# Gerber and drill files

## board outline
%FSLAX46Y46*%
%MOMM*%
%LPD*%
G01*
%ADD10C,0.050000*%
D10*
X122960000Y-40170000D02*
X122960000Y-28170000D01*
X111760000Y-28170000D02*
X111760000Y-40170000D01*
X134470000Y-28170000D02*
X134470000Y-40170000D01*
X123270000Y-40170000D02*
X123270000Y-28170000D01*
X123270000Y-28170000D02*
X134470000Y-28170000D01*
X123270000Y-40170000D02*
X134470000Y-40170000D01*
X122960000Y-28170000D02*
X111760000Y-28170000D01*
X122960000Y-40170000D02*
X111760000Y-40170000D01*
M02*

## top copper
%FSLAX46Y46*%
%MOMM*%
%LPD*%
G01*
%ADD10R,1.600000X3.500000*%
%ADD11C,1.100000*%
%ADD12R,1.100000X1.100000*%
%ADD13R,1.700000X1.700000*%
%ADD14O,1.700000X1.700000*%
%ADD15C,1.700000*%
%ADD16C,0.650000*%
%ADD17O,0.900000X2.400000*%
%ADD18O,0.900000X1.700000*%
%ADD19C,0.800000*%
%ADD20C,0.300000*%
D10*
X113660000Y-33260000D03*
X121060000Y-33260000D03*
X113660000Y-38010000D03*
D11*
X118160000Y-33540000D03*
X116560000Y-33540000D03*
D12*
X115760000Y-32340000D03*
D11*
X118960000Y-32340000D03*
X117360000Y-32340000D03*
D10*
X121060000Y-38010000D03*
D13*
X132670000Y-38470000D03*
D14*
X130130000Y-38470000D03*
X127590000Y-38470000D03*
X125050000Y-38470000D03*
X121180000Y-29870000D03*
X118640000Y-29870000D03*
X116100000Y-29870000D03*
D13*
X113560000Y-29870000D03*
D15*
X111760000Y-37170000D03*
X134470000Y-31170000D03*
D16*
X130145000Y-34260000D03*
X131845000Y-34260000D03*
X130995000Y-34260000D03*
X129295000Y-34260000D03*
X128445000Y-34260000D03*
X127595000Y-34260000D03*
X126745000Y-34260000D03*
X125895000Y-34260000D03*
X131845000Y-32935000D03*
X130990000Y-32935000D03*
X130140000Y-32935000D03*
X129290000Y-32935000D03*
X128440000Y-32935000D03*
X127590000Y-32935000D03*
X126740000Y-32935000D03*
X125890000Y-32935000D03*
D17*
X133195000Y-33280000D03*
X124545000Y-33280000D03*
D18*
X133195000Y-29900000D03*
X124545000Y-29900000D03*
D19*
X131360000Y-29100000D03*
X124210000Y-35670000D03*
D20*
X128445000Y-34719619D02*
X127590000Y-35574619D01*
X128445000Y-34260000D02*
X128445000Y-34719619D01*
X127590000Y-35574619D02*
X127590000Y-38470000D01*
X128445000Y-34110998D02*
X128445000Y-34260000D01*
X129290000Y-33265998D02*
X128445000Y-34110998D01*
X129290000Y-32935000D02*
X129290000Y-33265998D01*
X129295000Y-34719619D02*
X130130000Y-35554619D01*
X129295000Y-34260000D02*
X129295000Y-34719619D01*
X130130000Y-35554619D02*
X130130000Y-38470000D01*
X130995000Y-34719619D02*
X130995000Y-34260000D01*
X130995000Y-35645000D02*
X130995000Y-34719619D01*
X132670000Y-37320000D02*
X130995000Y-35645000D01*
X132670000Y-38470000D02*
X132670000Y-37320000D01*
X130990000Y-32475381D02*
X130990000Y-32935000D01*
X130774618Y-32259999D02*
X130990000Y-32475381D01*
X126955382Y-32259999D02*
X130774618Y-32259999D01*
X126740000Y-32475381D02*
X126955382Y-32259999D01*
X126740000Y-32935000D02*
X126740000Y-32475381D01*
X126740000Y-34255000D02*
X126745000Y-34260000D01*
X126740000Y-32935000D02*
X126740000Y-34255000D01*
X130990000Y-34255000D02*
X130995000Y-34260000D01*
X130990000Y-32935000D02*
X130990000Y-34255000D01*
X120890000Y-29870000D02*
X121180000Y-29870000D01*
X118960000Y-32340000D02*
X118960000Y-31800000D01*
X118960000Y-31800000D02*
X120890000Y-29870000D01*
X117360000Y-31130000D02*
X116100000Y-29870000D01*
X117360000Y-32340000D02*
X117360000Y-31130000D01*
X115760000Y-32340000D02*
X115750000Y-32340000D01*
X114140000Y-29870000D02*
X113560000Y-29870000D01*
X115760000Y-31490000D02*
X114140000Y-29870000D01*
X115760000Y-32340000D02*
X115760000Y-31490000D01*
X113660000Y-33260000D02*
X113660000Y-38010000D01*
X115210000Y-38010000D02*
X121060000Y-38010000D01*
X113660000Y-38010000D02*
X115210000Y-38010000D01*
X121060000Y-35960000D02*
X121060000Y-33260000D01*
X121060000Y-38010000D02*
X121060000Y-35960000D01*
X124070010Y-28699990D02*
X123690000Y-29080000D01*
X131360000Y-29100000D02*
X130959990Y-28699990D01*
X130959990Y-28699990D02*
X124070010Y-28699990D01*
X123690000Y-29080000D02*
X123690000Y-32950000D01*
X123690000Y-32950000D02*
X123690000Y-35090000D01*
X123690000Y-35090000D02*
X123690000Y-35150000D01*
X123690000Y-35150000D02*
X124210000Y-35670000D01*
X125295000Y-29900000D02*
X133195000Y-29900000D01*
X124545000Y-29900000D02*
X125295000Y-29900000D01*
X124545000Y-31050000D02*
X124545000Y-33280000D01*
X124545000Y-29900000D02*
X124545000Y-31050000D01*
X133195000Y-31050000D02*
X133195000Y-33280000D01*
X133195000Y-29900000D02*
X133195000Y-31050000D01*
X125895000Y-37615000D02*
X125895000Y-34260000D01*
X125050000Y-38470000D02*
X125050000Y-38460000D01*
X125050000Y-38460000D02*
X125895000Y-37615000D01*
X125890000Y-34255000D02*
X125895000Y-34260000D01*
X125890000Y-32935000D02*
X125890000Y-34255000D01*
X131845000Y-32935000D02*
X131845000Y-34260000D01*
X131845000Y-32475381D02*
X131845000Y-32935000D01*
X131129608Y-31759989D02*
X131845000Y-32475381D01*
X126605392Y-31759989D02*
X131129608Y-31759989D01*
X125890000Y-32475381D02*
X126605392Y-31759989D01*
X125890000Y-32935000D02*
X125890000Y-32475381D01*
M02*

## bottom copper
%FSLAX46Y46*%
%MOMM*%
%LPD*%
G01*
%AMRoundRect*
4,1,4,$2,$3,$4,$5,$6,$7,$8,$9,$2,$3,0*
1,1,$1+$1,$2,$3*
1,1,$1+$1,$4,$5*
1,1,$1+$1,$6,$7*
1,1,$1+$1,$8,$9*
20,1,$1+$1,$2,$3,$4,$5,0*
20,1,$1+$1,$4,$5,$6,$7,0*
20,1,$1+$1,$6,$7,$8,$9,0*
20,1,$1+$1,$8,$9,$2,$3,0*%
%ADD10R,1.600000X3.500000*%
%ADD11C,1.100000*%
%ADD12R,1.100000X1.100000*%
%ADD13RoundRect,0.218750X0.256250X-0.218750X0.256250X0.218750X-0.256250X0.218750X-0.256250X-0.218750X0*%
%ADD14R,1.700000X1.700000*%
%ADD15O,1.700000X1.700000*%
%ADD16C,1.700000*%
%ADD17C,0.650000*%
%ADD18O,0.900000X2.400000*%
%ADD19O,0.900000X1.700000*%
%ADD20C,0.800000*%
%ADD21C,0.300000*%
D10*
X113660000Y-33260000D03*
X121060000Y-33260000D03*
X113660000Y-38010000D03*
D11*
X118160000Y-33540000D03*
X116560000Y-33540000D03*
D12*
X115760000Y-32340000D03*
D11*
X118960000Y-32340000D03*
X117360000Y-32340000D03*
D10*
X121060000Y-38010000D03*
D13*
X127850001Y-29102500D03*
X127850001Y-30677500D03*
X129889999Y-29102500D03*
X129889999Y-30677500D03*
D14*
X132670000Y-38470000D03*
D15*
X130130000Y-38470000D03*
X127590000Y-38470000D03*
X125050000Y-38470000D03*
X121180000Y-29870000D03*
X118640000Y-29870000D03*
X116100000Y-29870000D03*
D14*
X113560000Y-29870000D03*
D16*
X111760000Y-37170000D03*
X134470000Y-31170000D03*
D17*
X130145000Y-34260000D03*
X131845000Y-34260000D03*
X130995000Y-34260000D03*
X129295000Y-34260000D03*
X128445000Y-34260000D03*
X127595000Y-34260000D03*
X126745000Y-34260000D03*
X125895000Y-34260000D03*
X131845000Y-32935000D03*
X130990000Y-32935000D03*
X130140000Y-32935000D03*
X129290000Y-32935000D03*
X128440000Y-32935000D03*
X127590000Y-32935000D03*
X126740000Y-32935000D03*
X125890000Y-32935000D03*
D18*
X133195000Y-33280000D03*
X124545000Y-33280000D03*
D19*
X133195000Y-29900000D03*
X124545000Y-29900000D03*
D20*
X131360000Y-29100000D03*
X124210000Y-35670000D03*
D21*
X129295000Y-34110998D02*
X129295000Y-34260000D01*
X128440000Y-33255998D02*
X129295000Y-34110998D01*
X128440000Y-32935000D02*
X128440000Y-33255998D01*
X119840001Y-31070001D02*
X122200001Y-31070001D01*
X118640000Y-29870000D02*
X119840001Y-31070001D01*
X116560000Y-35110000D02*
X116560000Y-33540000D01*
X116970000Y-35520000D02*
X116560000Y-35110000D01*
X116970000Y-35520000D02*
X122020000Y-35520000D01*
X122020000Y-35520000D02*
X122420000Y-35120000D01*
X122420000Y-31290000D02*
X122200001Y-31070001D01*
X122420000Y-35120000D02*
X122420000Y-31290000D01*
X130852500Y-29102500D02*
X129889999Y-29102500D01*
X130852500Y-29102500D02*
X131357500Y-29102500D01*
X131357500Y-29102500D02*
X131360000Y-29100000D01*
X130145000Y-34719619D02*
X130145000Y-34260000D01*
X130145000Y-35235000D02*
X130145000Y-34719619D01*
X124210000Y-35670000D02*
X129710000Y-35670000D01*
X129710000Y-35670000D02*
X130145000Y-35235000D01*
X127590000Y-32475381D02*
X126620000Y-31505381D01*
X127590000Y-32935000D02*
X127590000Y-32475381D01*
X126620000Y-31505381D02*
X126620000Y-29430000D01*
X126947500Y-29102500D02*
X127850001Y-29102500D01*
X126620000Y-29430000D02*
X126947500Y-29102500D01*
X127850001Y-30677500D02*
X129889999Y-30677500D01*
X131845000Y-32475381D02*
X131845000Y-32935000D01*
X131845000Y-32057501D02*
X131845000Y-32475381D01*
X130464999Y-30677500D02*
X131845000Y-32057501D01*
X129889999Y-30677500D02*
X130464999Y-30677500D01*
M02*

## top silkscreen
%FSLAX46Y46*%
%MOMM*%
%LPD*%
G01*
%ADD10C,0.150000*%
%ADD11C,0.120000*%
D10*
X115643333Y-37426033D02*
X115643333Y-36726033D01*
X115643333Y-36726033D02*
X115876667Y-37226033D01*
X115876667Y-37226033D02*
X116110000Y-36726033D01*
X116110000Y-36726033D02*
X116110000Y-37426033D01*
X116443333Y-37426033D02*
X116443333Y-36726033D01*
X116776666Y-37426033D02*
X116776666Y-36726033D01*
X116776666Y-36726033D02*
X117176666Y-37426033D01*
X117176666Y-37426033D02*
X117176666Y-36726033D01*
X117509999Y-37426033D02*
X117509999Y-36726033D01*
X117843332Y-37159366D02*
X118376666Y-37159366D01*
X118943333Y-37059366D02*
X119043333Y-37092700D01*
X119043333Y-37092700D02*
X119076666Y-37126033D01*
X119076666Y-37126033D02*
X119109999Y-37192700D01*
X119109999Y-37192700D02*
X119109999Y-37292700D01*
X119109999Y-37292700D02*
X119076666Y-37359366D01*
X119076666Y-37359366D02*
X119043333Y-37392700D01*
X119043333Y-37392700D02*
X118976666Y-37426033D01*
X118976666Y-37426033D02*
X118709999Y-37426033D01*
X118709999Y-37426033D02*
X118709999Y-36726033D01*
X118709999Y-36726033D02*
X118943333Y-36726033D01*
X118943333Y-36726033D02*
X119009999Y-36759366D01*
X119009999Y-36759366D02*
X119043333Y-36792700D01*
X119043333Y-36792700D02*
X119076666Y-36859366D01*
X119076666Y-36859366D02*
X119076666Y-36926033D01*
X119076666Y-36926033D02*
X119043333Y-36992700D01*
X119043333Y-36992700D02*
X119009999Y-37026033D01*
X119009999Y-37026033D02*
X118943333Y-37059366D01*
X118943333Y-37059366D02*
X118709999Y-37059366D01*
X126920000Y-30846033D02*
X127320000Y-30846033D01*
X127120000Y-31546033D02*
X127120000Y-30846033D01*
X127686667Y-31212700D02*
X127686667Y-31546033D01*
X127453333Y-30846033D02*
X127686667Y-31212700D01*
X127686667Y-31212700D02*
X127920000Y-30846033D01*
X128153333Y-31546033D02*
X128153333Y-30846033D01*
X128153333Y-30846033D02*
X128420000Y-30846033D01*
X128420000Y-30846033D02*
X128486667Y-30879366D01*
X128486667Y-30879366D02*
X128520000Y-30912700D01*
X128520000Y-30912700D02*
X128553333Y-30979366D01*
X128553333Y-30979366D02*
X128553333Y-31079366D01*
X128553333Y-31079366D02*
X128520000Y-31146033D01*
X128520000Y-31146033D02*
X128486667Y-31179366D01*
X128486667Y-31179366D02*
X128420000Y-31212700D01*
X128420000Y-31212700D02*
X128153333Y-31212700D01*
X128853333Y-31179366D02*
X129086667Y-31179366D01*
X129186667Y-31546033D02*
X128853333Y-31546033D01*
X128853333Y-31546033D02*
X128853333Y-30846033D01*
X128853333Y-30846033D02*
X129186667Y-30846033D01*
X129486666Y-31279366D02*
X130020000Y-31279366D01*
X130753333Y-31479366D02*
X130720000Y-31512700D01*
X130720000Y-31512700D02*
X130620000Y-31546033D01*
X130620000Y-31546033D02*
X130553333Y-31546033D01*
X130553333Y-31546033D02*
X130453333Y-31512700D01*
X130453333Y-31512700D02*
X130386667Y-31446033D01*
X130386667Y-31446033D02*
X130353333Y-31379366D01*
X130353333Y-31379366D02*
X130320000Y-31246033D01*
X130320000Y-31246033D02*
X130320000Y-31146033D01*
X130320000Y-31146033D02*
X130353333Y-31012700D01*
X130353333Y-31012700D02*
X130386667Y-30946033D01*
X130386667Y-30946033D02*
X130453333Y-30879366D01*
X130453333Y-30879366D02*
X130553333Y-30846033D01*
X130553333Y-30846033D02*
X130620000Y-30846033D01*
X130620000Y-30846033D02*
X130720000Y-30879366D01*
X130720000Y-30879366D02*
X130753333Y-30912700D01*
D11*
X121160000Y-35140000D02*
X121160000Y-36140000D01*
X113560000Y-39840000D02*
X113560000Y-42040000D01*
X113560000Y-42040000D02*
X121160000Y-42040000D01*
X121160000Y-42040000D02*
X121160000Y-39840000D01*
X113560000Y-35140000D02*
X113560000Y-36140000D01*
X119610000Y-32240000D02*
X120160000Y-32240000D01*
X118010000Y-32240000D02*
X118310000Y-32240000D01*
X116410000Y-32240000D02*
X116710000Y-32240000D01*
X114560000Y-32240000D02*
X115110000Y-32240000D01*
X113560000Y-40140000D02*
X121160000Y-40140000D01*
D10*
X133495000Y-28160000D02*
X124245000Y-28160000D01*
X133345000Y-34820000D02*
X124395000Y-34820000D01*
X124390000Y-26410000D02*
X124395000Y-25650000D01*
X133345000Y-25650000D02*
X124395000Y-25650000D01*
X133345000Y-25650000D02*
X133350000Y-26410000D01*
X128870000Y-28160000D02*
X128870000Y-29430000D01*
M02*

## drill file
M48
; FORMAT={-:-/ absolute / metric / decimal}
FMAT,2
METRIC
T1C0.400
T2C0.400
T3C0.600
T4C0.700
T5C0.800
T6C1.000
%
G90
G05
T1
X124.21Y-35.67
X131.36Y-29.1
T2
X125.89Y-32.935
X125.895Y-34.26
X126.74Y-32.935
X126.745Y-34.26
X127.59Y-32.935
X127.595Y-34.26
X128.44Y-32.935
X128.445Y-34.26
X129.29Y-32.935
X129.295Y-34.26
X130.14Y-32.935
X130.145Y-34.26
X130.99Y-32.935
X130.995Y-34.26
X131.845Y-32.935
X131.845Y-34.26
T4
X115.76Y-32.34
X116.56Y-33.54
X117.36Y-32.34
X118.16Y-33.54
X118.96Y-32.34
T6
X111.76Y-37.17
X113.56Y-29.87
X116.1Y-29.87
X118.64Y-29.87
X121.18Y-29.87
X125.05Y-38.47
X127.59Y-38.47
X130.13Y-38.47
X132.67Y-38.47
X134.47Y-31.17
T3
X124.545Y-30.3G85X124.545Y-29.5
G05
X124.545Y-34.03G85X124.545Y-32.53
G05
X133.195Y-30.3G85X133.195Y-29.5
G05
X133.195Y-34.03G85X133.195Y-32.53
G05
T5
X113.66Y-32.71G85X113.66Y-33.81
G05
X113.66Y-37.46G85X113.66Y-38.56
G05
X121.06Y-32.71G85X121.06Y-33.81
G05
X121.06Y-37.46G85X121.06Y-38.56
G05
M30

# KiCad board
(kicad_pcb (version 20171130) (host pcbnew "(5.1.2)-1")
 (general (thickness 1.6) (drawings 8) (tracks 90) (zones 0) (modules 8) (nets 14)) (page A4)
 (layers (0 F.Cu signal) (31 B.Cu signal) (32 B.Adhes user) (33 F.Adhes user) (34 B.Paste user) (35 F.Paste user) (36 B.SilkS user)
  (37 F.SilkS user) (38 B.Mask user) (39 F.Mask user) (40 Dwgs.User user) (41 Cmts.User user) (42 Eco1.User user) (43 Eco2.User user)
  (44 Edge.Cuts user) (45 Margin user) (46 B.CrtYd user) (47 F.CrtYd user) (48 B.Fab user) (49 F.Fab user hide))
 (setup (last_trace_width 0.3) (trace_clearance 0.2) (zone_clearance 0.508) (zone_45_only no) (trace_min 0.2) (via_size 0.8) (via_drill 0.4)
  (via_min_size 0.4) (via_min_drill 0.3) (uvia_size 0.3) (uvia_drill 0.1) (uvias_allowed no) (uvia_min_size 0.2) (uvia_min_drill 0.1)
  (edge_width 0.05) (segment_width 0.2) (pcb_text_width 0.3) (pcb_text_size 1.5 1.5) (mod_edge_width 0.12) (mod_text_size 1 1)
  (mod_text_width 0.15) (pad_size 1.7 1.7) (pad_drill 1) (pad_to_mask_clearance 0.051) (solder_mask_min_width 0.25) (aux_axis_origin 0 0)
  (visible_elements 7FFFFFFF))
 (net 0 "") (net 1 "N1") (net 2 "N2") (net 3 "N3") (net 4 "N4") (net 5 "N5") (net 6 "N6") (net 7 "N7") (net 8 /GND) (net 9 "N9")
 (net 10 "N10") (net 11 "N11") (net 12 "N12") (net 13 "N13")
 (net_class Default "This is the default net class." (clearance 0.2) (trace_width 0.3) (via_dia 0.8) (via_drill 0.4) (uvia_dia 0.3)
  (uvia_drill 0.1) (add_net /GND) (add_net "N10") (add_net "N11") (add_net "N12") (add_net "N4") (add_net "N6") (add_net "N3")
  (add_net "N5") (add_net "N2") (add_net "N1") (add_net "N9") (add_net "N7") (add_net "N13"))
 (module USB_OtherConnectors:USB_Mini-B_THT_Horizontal (layer F.Cu) (at 115.76 32.34)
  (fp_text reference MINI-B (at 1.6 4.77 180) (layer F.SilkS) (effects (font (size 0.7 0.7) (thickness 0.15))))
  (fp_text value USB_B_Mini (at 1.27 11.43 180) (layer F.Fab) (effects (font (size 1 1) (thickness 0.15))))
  (fp_line (start 5.4 2.8) (end 5.4 3.8) (layer F.SilkS) (width 0.12))
  (fp_line (start -2.2 7.5) (end -2.2 9.7) (layer F.SilkS) (width 0.12))
  (fp_line (start -2.2 9.7) (end 5.4 9.7) (layer F.SilkS) (width 0.12))
  (fp_line (start 5.4 9.7) (end 5.4 7.5) (layer F.SilkS) (width 0.12))
  (fp_line (start -2.2 2.8) (end -2.2 3.8) (layer F.SilkS) (width 0.12))
  (fp_line (start 3.85 -0.1) (end 4.4 -0.1) (layer F.SilkS) (width 0.12))
  (fp_line (start 2.25 -0.1) (end 2.55 -0.1) (layer F.SilkS) (width 0.12))
  (fp_line (start 0.65 -0.1) (end 0.95 -0.1) (layer F.SilkS) (width 0.12))
  (fp_line (start -1.2 -0.1) (end -0.65 -0.1) (layer F.SilkS) (width 0.12))
  (fp_line (start -2.2 7.8) (end 5.4 7.8) (layer F.SilkS) (width 0.12))
  (pad 6 thru_hole rect (at -2.1 0.92) (size 1.6 3.5) (drill oval 0.8 1.9) (layers *.Cu *.Mask) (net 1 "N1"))
  (pad 6 thru_hole rect (at 5.3 0.92) (size 1.6 3.5) (drill oval 0.8 1.9) (layers *.Cu *.Mask) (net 1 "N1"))
  (pad 6 thru_hole rect (at -2.1 5.67) (size 1.6 3.5) (drill oval 0.8 1.9) (layers *.Cu *.Mask) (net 1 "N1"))
  (pad 4 thru_hole circle (at 2.4 1.2) (size 1.1 1.1) (drill 0.7) (layers *.Cu *.Mask) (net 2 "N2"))
  (pad 2 thru_hole circle (at 0.8 1.2) (size 1.1 1.1) (drill 0.7) (layers *.Cu *.Mask) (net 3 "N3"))
  (pad 1 thru_hole rect (at 0 0) (size 1.1 1.1) (drill 0.7) (layers *.Cu *.Mask) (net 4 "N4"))
  (pad 5 thru_hole circle (at 3.2 0) (size 1.1 1.1) (drill 0.7) (layers *.Cu *.Mask) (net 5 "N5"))
  (pad 3 thru_hole circle (at 1.6 0) (size 1.1 1.1) (drill 0.7) (layers *.Cu *.Mask) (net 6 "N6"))
  (pad 6 thru_hole rect (at 5.3 5.67) (size 1.6 3.5) (drill oval 0.8 1.9) (layers *.Cu *.Mask) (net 1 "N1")))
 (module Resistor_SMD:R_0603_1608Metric (layer B.Cu) (at 127.850001 29.89 90)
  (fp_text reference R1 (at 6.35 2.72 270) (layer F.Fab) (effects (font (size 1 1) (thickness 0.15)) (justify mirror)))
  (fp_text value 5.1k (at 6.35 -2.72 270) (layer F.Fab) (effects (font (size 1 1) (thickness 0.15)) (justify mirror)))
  (pad 2 smd roundrect (at 0.7875 0 90) (size 0.875 0.95) (layers B.Cu B.Paste B.Mask) (roundrect_rratio 0.25) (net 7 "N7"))
  (pad 1 smd roundrect (at -0.7875 0 90) (size 0.875 0.95) (layers B.Cu B.Paste B.Mask) (roundrect_rratio 0.25) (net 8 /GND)))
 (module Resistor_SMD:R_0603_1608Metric (layer B.Cu) (at 129.889999 29.89 90)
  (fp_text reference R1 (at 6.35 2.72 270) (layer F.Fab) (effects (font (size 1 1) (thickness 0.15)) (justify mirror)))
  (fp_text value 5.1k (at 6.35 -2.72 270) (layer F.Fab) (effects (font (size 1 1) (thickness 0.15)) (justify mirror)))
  (pad 2 smd roundrect (at 0.7875 0 90) (size 0.875 0.95) (layers B.Cu B.Paste B.Mask) (roundrect_rratio 0.25) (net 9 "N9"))
  (pad 1 smd roundrect (at -0.7875 0 90) (size 0.875 0.95) (layers B.Cu B.Paste B.Mask) (roundrect_rratio 0.25) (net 8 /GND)))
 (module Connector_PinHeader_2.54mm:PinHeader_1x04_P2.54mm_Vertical (layer F.Cu) (at 132.67 38.47 270)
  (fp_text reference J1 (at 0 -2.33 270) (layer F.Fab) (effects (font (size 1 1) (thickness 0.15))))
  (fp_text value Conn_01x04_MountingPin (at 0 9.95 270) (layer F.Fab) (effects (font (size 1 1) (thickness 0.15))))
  (pad 1 thru_hole rect (at 0 0 270) (size 1.7 1.7) (drill 1) (layers *.Cu *.Mask) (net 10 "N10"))
  (pad 2 thru_hole oval (at 0 2.54 270) (size 1.7 1.7) (drill 1) (layers *.Cu *.Mask) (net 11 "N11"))
  (pad 3 thru_hole oval (at 0 5.08 270) (size 1.7 1.7) (drill 1) (layers *.Cu *.Mask) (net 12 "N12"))
  (pad 4 thru_hole oval (at 0 7.62 270) (size 1.7 1.7) (drill 1) (layers *.Cu *.Mask) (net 8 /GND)))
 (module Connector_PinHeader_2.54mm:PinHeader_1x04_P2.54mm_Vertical (layer F.Cu) (at 113.56 29.87 90)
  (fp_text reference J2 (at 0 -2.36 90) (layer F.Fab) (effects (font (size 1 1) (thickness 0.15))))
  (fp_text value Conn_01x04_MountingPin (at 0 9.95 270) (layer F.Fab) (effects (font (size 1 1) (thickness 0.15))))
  (pad 4 thru_hole oval (at 0 7.62 90) (size 1.7 1.7) (drill 1) (layers *.Cu *.Mask) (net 5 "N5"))
  (pad 3 thru_hole oval (at 0 5.08 90) (size 1.7 1.7) (drill 1) (layers *.Cu *.Mask) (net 3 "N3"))
  (pad 2 thru_hole oval (at 0 2.54 90) (size 1.7 1.7) (drill 1) (layers *.Cu *.Mask) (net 6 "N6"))
  (pad 1 thru_hole rect (at 0 0 90) (size 1.7 1.7) (drill 1) (layers *.Cu *.Mask) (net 4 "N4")))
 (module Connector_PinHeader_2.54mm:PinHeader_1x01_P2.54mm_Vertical (layer F.Cu) (at 111.76 37.17 180)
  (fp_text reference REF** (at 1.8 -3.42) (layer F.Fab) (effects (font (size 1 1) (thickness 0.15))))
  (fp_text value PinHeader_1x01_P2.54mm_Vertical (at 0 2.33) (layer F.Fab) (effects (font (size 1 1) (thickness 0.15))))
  (pad 1 thru_hole circle (at 0 0 180) (size 1.7 1.7) (drill 1) (layers *.Cu *.Mask)))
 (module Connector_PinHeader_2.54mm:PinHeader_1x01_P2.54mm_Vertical (layer F.Cu) (at 134.47 31.17)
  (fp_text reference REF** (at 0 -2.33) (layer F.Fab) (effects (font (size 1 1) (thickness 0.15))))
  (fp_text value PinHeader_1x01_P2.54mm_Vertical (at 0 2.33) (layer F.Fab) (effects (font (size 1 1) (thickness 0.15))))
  (pad 1 thru_hole circle (at 0 0) (size 1.7 1.7) (drill 1) (layers *.Cu *.Mask)))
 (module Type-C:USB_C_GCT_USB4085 (layer F.Cu) (at 128.87 28.16 180)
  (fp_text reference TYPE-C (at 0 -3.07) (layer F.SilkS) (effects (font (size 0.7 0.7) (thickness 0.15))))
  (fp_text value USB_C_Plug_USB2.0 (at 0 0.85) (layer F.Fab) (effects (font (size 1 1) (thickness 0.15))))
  (fp_line (start -4.625 0) (end 4.625 0) (layer F.SilkS) (width 0.15))
  (fp_line (start -4.475 -6.66) (end 4.475 -6.66) (layer F.SilkS) (width 0.15))
  (fp_line (start 4.48 1.75) (end 4.475 2.51) (layer F.SilkS) (width 0.15))
  (fp_line (start -4.475 2.51) (end 4.475 2.51) (layer F.SilkS) (width 0.15))
  (fp_line (start -4.475 2.51) (end -4.48 1.75) (layer F.SilkS) (width 0.15))
  (fp_line (start 0 0) (end 0 -1.27) (layer F.SilkS) (width 0.15))
  (pad A5 thru_hole circle (at -1.275 -6.1 180) (size 0.65 0.65) (drill 0.4) (layers *.Cu *.Mask) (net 9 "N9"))
  (pad A1 thru_hole circle (at -2.975 -6.1 180) (size 0.65 0.65) (drill 0.4) (layers *.Cu *.Mask) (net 8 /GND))
  (pad A4 thru_hole circle (at -2.125 -6.1 180) (size 0.65 0.65) (drill 0.4) (layers *.Cu *.Mask) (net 10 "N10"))
  (pad A6 thru_hole circle (at -0.425 -6.1 180) (size 0.65 0.65) (drill 0.4) (layers *.Cu *.Mask) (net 11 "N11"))
  (pad A7 thru_hole circle (at 0.425 -6.1 180) (size 0.65 0.65) (drill 0.4) (layers *.Cu *.Mask) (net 12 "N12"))
  (pad A8 thru_hole circle (at 1.275 -6.1 180) (size 0.65 0.65) (drill 0.4) (layers *.Cu *.Mask))
  (pad A9 thru_hole circle (at 2.125 -6.1 180) (size 0.65 0.65) (drill 0.4) (layers *.Cu *.Mask) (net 10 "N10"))
  (pad A12 thru_hole circle (at 2.975 -6.1 180) (size 0.65 0.65) (drill 0.4) (layers *.Cu *.Mask) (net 8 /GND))
  (pad B12 thru_hole circle (at -2.975 -4.775 180) (size 0.65 0.65) (drill 0.4) (layers *.Cu *.Mask) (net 8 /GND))
  (pad B9 thru_hole circle (at -2.12 -4.775 180) (size 0.65 0.65) (drill 0.4) (layers *.Cu *.Mask) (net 10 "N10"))
  (pad B8 thru_hole circle (at -1.27 -4.775 180) (size 0.65 0.65) (drill 0.4) (layers *.Cu *.Mask))
  (pad B7 thru_hole circle (at -0.42 -4.775 180) (size 0.65 0.65) (drill 0.4) (layers *.Cu *.Mask) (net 12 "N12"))
  (pad B6 thru_hole circle (at 0.43 -4.775 180) (size 0.65 0.65) (drill 0.4) (layers *.Cu *.Mask) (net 11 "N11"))
  (pad B5 thru_hole circle (at 1.28 -4.775 180) (size 0.65 0.65) (drill 0.4) (layers *.Cu *.Mask) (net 7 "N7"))
  (pad B4 thru_hole circle (at 2.13 -4.775 180) (size 0.65 0.65) (drill 0.4) (layers *.Cu *.Mask) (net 10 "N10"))
  (pad B1 thru_hole circle (at 2.98 -4.775 180) (size 0.65 0.65) (drill 0.4) (layers *.Cu *.Mask) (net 8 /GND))
  (pad S1 thru_hole oval (at -4.325 -5.12 180) (size 0.9 2.4) (drill oval 0.6 2.1) (layers *.Cu *.Mask) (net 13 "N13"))
  (pad S1 thru_hole oval (at 4.325 -5.12 180) (size 0.9 2.4) (drill oval 0.6 2.1) (layers *.Cu *.Mask) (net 13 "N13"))
  (pad S1 thru_hole oval (at -4.325 -1.74 180) (size 0.9 1.7) (drill oval 0.6 1.4) (layers *.Cu *.Mask) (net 13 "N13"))
  (pad S1 thru_hole oval (at 4.325 -1.74 180) (size 0.9 1.7) (drill oval 0.6 1.4) (layers *.Cu *.Mask) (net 13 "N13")))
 (gr_line (start 122.96 40.17) (end 122.96 28.17) (layer Edge.Cuts) (width 0.05))
 (gr_line (start 111.76 28.17) (end 111.76 40.17) (layer Edge.Cuts) (width 0.05))
 (gr_line (start 134.47 28.17) (end 134.47 40.17) (layer Edge.Cuts) (width 0.05))
 (gr_line (start 123.27 40.17) (end 123.27 28.17) (layer Edge.Cuts) (width 0.05))
 (gr_line (start 123.27 28.17) (end 134.47 28.17) (layer Edge.Cuts) (width 0.05))
 (gr_line (start 123.27 40.17) (end 134.47 40.17) (layer Edge.Cuts) (width 0.05))
 (gr_line (start 122.96 28.17) (end 111.76 28.17) (layer Edge.Cuts) (width 0.05))
 (gr_line (start 122.96 40.17) (end 111.76 40.17) (layer Edge.Cuts) (width 0.05))
 (segment (start 128.445 34.719619) (end 127.59 35.574619) (width 0.3) (layer F.Cu) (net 12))
 (segment (start 128.445 34.26) (end 128.445 34.719619) (width 0.3) (layer F.Cu) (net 12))
 (segment (start 127.59 35.574619) (end 127.59 38.47) (width 0.3) (layer F.Cu) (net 12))
 (segment (start 128.445 34.110998) (end 128.445 34.26) (width 0.3) (layer F.Cu) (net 12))
 (segment (start 129.29 33.265998) (end 128.445 34.110998) (width 0.3) (layer F.Cu) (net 12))
 (segment (start 129.29 32.935) (end 129.29 33.265998) (width 0.3) (layer F.Cu) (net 12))
 (segment (start 129.295 34.719619) (end 130.13 35.554619) (width 0.3) (layer F.Cu) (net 11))
 (segment (start 129.295 34.26) (end 129.295 34.719619) (width 0.3) (layer F.Cu) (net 11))
 (segment (start 130.13 35.554619) (end 130.13 38.47) (width 0.3) (layer F.Cu) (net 11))
 (segment (start 129.295 34.110998) (end 129.295 34.26) (width 0.3) (layer B.Cu) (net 11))
 (segment (start 128.44 33.255998) (end 129.295 34.110998) (width 0.3) (layer B.Cu) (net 11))
 (segment (start 128.44 32.935) (end 128.44 33.255998) (width 0.3) (layer B.Cu) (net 11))
 (segment (start 130.995 34.719619) (end 130.995 34.26) (width 0.3) (layer F.Cu) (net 10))
 (segment (start 130.995 35.645) (end 130.995 34.719619) (width 0.3) (layer F.Cu) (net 10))
 (segment (start 132.67 37.32) (end 130.995 35.645) (width 0.3) (layer F.Cu) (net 10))
 (segment (start 132.67 38.47) (end 132.67 37.32) (width 0.3) (layer F.Cu) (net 10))
 (segment (start 130.99 32.475381) (end 130.99 32.935) (width 0.3) (layer F.Cu) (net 10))
 (segment (start 130.774618 32.259999) (end 130.99 32.475381) (width 0.3) (layer F.Cu) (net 10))
 (segment (start 126.955382 32.259999) (end 130.774618 32.259999) (width 0.3) (layer F.Cu) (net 10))
 (segment (start 126.74 32.475381) (end 126.955382 32.259999) (width 0.3) (layer F.Cu) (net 10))
 (segment (start 126.74 32.935) (end 126.74 32.475381) (width 0.3) (layer F.Cu) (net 10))
 (segment (start 126.74 34.255) (end 126.745 34.26) (width 0.3) (layer F.Cu) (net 10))
 (segment (start 126.74 32.935) (end 126.74 34.255) (width 0.3) (layer F.Cu) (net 10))
 (segment (start 130.99 34.255) (end 130.995 34.26) (width 0.3) (layer F.Cu) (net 10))
 (segment (start 130.99 32.935) (end 130.99 34.255) (width 0.3) (layer F.Cu) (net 10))
 (segment (start 120.89 29.87) (end 121.18 29.87) (width 0.3) (layer F.Cu) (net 5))
 (segment (start 118.96 32.34) (end 118.96 31.8) (width 0.3) (layer F.Cu) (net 5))
 (segment (start 118.96 31.8) (end 120.89 29.87) (width 0.3) (layer F.Cu) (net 5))
 (segment (start 119.840001 31.070001) (end 122.200001 31.070001) (width 0.3) (layer B.Cu) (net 3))
 (segment (start 118.64 29.87) (end 119.840001 31.070001) (width 0.3) (layer B.Cu) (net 3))
 (segment (start 116.56 35.11) (end 116.56 33.54) (width 0.3) (layer B.Cu) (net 3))
 (segment (start 116.97 35.52) (end 116.56 35.11) (width 0.3) (layer B.Cu) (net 3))
 (segment (start 116.97 35.52) (end 122.02 35.52) (width 0.3) (layer B.Cu) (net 3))
 (segment (start 122.02 35.52) (end 122.42 35.12) (width 0.3) (layer B.Cu) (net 3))
 (segment (start 122.42 31.29) (end 122.200001 31.070001) (width 0.3) (layer B.Cu) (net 3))
 (segment (start 122.42 35.12) (end 122.42 31.29) (width 0.3) (layer B.Cu) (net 3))
 (segment (start 117.36 31.13) (end 116.1 29.87) (width 0.3) (layer F.Cu) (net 6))
 (segment (start 117.36 32.34) (end 117.36 31.13) (width 0.3) (layer F.Cu) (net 6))
 (segment (start 115.76 32.34) (end 115.75 32.34) (width 0.3) (layer F.Cu) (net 4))
 (segment (start 114.14 29.87) (end 113.56 29.87) (width 0.3) (layer F.Cu) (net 4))
 (segment (start 115.76 31.49) (end 114.14 29.87) (width 0.3) (layer F.Cu) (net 4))
 (segment (start 115.76 32.34) (end 115.76 31.49) (width 0.3) (layer F.Cu) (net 4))
 (segment (start 113.66 33.26) (end 113.66 38.01) (width 0.3) (layer F.Cu) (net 1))
 (segment (start 115.21 38.01) (end 121.06 38.01) (width 0.3) (layer F.Cu) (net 1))
 (segment (start 113.66 38.01) (end 115.21 38.01) (width 0.3) (layer F.Cu) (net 1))
 (segment (start 121.06 35.96) (end 121.06 33.26) (width 0.3) (layer F.Cu) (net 1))
 (segment (start 121.06 38.01) (end 121.06 35.96) (width 0.3) (layer F.Cu) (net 1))
 (segment (start 130.8525 29.1025) (end 129.889999 29.1025) (width 0.3) (layer B.Cu) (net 9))
 (via (at 131.36 29.1) (size 0.8) (drill 0.4) (layers F.Cu B.Cu) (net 9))
 (segment (start 130.8525 29.1025) (end 131.3575 29.1025) (width 0.3) (layer B.Cu) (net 9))
 (segment (start 131.3575 29.1025) (end 131.36 29.1) (width 0.3) (layer B.Cu) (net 9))
 (segment (start 124.07001 28.69999) (end 123.69 29.08) (width 0.3) (layer F.Cu) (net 9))
 (segment (start 131.36 29.1) (end 130.95999 28.69999) (width 0.3) (layer F.Cu) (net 9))
 (segment (start 130.95999 28.69999) (end 124.07001 28.69999) (width 0.3) (layer F.Cu) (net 9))
 (segment (start 123.69 29.08) (end 123.69 32.95) (width 0.3) (layer F.Cu) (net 9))
 (segment (start 123.69 32.95) (end 123.69 35.09) (width 0.3) (layer F.Cu) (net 9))
 (segment (start 123.69 35.09) (end 123.69 35.15) (width 0.3) (layer F.Cu) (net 9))
 (segment (start 123.69 35.15) (end 124.21 35.67) (width 0.3) (layer F.Cu) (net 9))
 (via (at 124.21 35.67) (size 0.8) (drill 0.4) (layers F.Cu B.Cu) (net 9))
 (segment (start 130.145 34.719619) (end 130.145 34.26) (width 0.3) (layer B.Cu) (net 9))
 (segment (start 130.145 35.235) (end 130.145 34.719619) (width 0.3) (layer B.Cu) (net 9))
 (segment (start 124.21 35.67) (end 129.71 35.67) (width 0.3) (layer B.Cu) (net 9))
 (segment (start 129.71 35.67) (end 130.145 35.235) (width 0.3) (layer B.Cu) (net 9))
 (segment (start 127.59 32.475381) (end 126.62 31.505381) (width 0.3) (layer B.Cu) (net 7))
 (segment (start 127.59 32.935) (end 127.59 32.475381) (width 0.3) (layer B.Cu) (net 7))
 (segment (start 126.62 31.505381) (end 126.62 29.43) (width 0.3) (layer B.Cu) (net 7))
 (segment (start 126.9475 29.1025) (end 127.850001 29.1025) (width 0.3) (layer B.Cu) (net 7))
 (segment (start 126.62 29.43) (end 126.9475 29.1025) (width 0.3) (layer B.Cu) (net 7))
 (segment (start 125.295 29.9) (end 133.195 29.9) (width 0.3) (layer F.Cu) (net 13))
 (segment (start 124.545 29.9) (end 125.295 29.9) (width 0.3) (layer F.Cu) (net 13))
 (segment (start 124.545 31.05) (end 124.545 33.28) (width 0.3) (layer F.Cu) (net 13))
 (segment (start 124.545 29.9) (end 124.545 31.05) (width 0.3) (layer F.Cu) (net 13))
 (segment (start 133.195 31.05) (end 133.195 33.28) (width 0.3) (layer F.Cu) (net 13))
 (segment (start 133.195 29.9) (end 133.195 31.05) (width 0.3) (layer F.Cu) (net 13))
 (segment (start 125.895 37.615) (end 125.895 34.26) (width 0.3) (layer F.Cu) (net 8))
 (segment (start 125.05 38.47) (end 125.05 38.46) (width 0.3) (layer F.Cu) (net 8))
 (segment (start 125.05 38.46) (end 125.895 37.615) (width 0.3) (layer F.Cu) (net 8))
 (segment (start 125.89 34.255) (end 125.895 34.26) (width 0.3) (layer F.Cu) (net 8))
 (segment (start 125.89 32.935) (end 125.89 34.255) (width 0.3) (layer F.Cu) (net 8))
 (segment (start 131.845 32.935) (end 131.845 34.26) (width 0.3) (layer F.Cu) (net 8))
 (segment (start 131.845 32.475381) (end 131.845 32.935) (width 0.3) (layer F.Cu) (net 8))
 (segment (start 131.129608 31.759989) (end 131.845 32.475381) (width 0.3) (layer F.Cu) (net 8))
 (segment (start 126.605392 31.759989) (end 131.129608 31.759989) (width 0.3) (layer F.Cu) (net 8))
 (segment (start 125.89 32.475381) (end 126.605392 31.759989) (width 0.3) (layer F.Cu) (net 8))
 (segment (start 125.89 32.935) (end 125.89 32.475381) (width 0.3) (layer F.Cu) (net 8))
 (segment (start 127.850001 30.6775) (end 129.889999 30.6775) (width 0.3) (layer B.Cu) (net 8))
 (segment (start 131.845 32.475381) (end 131.845 32.935) (width 0.3) (layer B.Cu) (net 8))
 (segment (start 131.845 32.057501) (end 131.845 32.475381) (width 0.3) (layer B.Cu) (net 8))
 (segment (start 130.464999 30.6775) (end 131.845 32.057501) (width 0.3) (layer B.Cu) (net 8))
 (segment (start 129.889999 30.6775) (end 130.464999 30.6775) (width 0.3) (layer B.Cu) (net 8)))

